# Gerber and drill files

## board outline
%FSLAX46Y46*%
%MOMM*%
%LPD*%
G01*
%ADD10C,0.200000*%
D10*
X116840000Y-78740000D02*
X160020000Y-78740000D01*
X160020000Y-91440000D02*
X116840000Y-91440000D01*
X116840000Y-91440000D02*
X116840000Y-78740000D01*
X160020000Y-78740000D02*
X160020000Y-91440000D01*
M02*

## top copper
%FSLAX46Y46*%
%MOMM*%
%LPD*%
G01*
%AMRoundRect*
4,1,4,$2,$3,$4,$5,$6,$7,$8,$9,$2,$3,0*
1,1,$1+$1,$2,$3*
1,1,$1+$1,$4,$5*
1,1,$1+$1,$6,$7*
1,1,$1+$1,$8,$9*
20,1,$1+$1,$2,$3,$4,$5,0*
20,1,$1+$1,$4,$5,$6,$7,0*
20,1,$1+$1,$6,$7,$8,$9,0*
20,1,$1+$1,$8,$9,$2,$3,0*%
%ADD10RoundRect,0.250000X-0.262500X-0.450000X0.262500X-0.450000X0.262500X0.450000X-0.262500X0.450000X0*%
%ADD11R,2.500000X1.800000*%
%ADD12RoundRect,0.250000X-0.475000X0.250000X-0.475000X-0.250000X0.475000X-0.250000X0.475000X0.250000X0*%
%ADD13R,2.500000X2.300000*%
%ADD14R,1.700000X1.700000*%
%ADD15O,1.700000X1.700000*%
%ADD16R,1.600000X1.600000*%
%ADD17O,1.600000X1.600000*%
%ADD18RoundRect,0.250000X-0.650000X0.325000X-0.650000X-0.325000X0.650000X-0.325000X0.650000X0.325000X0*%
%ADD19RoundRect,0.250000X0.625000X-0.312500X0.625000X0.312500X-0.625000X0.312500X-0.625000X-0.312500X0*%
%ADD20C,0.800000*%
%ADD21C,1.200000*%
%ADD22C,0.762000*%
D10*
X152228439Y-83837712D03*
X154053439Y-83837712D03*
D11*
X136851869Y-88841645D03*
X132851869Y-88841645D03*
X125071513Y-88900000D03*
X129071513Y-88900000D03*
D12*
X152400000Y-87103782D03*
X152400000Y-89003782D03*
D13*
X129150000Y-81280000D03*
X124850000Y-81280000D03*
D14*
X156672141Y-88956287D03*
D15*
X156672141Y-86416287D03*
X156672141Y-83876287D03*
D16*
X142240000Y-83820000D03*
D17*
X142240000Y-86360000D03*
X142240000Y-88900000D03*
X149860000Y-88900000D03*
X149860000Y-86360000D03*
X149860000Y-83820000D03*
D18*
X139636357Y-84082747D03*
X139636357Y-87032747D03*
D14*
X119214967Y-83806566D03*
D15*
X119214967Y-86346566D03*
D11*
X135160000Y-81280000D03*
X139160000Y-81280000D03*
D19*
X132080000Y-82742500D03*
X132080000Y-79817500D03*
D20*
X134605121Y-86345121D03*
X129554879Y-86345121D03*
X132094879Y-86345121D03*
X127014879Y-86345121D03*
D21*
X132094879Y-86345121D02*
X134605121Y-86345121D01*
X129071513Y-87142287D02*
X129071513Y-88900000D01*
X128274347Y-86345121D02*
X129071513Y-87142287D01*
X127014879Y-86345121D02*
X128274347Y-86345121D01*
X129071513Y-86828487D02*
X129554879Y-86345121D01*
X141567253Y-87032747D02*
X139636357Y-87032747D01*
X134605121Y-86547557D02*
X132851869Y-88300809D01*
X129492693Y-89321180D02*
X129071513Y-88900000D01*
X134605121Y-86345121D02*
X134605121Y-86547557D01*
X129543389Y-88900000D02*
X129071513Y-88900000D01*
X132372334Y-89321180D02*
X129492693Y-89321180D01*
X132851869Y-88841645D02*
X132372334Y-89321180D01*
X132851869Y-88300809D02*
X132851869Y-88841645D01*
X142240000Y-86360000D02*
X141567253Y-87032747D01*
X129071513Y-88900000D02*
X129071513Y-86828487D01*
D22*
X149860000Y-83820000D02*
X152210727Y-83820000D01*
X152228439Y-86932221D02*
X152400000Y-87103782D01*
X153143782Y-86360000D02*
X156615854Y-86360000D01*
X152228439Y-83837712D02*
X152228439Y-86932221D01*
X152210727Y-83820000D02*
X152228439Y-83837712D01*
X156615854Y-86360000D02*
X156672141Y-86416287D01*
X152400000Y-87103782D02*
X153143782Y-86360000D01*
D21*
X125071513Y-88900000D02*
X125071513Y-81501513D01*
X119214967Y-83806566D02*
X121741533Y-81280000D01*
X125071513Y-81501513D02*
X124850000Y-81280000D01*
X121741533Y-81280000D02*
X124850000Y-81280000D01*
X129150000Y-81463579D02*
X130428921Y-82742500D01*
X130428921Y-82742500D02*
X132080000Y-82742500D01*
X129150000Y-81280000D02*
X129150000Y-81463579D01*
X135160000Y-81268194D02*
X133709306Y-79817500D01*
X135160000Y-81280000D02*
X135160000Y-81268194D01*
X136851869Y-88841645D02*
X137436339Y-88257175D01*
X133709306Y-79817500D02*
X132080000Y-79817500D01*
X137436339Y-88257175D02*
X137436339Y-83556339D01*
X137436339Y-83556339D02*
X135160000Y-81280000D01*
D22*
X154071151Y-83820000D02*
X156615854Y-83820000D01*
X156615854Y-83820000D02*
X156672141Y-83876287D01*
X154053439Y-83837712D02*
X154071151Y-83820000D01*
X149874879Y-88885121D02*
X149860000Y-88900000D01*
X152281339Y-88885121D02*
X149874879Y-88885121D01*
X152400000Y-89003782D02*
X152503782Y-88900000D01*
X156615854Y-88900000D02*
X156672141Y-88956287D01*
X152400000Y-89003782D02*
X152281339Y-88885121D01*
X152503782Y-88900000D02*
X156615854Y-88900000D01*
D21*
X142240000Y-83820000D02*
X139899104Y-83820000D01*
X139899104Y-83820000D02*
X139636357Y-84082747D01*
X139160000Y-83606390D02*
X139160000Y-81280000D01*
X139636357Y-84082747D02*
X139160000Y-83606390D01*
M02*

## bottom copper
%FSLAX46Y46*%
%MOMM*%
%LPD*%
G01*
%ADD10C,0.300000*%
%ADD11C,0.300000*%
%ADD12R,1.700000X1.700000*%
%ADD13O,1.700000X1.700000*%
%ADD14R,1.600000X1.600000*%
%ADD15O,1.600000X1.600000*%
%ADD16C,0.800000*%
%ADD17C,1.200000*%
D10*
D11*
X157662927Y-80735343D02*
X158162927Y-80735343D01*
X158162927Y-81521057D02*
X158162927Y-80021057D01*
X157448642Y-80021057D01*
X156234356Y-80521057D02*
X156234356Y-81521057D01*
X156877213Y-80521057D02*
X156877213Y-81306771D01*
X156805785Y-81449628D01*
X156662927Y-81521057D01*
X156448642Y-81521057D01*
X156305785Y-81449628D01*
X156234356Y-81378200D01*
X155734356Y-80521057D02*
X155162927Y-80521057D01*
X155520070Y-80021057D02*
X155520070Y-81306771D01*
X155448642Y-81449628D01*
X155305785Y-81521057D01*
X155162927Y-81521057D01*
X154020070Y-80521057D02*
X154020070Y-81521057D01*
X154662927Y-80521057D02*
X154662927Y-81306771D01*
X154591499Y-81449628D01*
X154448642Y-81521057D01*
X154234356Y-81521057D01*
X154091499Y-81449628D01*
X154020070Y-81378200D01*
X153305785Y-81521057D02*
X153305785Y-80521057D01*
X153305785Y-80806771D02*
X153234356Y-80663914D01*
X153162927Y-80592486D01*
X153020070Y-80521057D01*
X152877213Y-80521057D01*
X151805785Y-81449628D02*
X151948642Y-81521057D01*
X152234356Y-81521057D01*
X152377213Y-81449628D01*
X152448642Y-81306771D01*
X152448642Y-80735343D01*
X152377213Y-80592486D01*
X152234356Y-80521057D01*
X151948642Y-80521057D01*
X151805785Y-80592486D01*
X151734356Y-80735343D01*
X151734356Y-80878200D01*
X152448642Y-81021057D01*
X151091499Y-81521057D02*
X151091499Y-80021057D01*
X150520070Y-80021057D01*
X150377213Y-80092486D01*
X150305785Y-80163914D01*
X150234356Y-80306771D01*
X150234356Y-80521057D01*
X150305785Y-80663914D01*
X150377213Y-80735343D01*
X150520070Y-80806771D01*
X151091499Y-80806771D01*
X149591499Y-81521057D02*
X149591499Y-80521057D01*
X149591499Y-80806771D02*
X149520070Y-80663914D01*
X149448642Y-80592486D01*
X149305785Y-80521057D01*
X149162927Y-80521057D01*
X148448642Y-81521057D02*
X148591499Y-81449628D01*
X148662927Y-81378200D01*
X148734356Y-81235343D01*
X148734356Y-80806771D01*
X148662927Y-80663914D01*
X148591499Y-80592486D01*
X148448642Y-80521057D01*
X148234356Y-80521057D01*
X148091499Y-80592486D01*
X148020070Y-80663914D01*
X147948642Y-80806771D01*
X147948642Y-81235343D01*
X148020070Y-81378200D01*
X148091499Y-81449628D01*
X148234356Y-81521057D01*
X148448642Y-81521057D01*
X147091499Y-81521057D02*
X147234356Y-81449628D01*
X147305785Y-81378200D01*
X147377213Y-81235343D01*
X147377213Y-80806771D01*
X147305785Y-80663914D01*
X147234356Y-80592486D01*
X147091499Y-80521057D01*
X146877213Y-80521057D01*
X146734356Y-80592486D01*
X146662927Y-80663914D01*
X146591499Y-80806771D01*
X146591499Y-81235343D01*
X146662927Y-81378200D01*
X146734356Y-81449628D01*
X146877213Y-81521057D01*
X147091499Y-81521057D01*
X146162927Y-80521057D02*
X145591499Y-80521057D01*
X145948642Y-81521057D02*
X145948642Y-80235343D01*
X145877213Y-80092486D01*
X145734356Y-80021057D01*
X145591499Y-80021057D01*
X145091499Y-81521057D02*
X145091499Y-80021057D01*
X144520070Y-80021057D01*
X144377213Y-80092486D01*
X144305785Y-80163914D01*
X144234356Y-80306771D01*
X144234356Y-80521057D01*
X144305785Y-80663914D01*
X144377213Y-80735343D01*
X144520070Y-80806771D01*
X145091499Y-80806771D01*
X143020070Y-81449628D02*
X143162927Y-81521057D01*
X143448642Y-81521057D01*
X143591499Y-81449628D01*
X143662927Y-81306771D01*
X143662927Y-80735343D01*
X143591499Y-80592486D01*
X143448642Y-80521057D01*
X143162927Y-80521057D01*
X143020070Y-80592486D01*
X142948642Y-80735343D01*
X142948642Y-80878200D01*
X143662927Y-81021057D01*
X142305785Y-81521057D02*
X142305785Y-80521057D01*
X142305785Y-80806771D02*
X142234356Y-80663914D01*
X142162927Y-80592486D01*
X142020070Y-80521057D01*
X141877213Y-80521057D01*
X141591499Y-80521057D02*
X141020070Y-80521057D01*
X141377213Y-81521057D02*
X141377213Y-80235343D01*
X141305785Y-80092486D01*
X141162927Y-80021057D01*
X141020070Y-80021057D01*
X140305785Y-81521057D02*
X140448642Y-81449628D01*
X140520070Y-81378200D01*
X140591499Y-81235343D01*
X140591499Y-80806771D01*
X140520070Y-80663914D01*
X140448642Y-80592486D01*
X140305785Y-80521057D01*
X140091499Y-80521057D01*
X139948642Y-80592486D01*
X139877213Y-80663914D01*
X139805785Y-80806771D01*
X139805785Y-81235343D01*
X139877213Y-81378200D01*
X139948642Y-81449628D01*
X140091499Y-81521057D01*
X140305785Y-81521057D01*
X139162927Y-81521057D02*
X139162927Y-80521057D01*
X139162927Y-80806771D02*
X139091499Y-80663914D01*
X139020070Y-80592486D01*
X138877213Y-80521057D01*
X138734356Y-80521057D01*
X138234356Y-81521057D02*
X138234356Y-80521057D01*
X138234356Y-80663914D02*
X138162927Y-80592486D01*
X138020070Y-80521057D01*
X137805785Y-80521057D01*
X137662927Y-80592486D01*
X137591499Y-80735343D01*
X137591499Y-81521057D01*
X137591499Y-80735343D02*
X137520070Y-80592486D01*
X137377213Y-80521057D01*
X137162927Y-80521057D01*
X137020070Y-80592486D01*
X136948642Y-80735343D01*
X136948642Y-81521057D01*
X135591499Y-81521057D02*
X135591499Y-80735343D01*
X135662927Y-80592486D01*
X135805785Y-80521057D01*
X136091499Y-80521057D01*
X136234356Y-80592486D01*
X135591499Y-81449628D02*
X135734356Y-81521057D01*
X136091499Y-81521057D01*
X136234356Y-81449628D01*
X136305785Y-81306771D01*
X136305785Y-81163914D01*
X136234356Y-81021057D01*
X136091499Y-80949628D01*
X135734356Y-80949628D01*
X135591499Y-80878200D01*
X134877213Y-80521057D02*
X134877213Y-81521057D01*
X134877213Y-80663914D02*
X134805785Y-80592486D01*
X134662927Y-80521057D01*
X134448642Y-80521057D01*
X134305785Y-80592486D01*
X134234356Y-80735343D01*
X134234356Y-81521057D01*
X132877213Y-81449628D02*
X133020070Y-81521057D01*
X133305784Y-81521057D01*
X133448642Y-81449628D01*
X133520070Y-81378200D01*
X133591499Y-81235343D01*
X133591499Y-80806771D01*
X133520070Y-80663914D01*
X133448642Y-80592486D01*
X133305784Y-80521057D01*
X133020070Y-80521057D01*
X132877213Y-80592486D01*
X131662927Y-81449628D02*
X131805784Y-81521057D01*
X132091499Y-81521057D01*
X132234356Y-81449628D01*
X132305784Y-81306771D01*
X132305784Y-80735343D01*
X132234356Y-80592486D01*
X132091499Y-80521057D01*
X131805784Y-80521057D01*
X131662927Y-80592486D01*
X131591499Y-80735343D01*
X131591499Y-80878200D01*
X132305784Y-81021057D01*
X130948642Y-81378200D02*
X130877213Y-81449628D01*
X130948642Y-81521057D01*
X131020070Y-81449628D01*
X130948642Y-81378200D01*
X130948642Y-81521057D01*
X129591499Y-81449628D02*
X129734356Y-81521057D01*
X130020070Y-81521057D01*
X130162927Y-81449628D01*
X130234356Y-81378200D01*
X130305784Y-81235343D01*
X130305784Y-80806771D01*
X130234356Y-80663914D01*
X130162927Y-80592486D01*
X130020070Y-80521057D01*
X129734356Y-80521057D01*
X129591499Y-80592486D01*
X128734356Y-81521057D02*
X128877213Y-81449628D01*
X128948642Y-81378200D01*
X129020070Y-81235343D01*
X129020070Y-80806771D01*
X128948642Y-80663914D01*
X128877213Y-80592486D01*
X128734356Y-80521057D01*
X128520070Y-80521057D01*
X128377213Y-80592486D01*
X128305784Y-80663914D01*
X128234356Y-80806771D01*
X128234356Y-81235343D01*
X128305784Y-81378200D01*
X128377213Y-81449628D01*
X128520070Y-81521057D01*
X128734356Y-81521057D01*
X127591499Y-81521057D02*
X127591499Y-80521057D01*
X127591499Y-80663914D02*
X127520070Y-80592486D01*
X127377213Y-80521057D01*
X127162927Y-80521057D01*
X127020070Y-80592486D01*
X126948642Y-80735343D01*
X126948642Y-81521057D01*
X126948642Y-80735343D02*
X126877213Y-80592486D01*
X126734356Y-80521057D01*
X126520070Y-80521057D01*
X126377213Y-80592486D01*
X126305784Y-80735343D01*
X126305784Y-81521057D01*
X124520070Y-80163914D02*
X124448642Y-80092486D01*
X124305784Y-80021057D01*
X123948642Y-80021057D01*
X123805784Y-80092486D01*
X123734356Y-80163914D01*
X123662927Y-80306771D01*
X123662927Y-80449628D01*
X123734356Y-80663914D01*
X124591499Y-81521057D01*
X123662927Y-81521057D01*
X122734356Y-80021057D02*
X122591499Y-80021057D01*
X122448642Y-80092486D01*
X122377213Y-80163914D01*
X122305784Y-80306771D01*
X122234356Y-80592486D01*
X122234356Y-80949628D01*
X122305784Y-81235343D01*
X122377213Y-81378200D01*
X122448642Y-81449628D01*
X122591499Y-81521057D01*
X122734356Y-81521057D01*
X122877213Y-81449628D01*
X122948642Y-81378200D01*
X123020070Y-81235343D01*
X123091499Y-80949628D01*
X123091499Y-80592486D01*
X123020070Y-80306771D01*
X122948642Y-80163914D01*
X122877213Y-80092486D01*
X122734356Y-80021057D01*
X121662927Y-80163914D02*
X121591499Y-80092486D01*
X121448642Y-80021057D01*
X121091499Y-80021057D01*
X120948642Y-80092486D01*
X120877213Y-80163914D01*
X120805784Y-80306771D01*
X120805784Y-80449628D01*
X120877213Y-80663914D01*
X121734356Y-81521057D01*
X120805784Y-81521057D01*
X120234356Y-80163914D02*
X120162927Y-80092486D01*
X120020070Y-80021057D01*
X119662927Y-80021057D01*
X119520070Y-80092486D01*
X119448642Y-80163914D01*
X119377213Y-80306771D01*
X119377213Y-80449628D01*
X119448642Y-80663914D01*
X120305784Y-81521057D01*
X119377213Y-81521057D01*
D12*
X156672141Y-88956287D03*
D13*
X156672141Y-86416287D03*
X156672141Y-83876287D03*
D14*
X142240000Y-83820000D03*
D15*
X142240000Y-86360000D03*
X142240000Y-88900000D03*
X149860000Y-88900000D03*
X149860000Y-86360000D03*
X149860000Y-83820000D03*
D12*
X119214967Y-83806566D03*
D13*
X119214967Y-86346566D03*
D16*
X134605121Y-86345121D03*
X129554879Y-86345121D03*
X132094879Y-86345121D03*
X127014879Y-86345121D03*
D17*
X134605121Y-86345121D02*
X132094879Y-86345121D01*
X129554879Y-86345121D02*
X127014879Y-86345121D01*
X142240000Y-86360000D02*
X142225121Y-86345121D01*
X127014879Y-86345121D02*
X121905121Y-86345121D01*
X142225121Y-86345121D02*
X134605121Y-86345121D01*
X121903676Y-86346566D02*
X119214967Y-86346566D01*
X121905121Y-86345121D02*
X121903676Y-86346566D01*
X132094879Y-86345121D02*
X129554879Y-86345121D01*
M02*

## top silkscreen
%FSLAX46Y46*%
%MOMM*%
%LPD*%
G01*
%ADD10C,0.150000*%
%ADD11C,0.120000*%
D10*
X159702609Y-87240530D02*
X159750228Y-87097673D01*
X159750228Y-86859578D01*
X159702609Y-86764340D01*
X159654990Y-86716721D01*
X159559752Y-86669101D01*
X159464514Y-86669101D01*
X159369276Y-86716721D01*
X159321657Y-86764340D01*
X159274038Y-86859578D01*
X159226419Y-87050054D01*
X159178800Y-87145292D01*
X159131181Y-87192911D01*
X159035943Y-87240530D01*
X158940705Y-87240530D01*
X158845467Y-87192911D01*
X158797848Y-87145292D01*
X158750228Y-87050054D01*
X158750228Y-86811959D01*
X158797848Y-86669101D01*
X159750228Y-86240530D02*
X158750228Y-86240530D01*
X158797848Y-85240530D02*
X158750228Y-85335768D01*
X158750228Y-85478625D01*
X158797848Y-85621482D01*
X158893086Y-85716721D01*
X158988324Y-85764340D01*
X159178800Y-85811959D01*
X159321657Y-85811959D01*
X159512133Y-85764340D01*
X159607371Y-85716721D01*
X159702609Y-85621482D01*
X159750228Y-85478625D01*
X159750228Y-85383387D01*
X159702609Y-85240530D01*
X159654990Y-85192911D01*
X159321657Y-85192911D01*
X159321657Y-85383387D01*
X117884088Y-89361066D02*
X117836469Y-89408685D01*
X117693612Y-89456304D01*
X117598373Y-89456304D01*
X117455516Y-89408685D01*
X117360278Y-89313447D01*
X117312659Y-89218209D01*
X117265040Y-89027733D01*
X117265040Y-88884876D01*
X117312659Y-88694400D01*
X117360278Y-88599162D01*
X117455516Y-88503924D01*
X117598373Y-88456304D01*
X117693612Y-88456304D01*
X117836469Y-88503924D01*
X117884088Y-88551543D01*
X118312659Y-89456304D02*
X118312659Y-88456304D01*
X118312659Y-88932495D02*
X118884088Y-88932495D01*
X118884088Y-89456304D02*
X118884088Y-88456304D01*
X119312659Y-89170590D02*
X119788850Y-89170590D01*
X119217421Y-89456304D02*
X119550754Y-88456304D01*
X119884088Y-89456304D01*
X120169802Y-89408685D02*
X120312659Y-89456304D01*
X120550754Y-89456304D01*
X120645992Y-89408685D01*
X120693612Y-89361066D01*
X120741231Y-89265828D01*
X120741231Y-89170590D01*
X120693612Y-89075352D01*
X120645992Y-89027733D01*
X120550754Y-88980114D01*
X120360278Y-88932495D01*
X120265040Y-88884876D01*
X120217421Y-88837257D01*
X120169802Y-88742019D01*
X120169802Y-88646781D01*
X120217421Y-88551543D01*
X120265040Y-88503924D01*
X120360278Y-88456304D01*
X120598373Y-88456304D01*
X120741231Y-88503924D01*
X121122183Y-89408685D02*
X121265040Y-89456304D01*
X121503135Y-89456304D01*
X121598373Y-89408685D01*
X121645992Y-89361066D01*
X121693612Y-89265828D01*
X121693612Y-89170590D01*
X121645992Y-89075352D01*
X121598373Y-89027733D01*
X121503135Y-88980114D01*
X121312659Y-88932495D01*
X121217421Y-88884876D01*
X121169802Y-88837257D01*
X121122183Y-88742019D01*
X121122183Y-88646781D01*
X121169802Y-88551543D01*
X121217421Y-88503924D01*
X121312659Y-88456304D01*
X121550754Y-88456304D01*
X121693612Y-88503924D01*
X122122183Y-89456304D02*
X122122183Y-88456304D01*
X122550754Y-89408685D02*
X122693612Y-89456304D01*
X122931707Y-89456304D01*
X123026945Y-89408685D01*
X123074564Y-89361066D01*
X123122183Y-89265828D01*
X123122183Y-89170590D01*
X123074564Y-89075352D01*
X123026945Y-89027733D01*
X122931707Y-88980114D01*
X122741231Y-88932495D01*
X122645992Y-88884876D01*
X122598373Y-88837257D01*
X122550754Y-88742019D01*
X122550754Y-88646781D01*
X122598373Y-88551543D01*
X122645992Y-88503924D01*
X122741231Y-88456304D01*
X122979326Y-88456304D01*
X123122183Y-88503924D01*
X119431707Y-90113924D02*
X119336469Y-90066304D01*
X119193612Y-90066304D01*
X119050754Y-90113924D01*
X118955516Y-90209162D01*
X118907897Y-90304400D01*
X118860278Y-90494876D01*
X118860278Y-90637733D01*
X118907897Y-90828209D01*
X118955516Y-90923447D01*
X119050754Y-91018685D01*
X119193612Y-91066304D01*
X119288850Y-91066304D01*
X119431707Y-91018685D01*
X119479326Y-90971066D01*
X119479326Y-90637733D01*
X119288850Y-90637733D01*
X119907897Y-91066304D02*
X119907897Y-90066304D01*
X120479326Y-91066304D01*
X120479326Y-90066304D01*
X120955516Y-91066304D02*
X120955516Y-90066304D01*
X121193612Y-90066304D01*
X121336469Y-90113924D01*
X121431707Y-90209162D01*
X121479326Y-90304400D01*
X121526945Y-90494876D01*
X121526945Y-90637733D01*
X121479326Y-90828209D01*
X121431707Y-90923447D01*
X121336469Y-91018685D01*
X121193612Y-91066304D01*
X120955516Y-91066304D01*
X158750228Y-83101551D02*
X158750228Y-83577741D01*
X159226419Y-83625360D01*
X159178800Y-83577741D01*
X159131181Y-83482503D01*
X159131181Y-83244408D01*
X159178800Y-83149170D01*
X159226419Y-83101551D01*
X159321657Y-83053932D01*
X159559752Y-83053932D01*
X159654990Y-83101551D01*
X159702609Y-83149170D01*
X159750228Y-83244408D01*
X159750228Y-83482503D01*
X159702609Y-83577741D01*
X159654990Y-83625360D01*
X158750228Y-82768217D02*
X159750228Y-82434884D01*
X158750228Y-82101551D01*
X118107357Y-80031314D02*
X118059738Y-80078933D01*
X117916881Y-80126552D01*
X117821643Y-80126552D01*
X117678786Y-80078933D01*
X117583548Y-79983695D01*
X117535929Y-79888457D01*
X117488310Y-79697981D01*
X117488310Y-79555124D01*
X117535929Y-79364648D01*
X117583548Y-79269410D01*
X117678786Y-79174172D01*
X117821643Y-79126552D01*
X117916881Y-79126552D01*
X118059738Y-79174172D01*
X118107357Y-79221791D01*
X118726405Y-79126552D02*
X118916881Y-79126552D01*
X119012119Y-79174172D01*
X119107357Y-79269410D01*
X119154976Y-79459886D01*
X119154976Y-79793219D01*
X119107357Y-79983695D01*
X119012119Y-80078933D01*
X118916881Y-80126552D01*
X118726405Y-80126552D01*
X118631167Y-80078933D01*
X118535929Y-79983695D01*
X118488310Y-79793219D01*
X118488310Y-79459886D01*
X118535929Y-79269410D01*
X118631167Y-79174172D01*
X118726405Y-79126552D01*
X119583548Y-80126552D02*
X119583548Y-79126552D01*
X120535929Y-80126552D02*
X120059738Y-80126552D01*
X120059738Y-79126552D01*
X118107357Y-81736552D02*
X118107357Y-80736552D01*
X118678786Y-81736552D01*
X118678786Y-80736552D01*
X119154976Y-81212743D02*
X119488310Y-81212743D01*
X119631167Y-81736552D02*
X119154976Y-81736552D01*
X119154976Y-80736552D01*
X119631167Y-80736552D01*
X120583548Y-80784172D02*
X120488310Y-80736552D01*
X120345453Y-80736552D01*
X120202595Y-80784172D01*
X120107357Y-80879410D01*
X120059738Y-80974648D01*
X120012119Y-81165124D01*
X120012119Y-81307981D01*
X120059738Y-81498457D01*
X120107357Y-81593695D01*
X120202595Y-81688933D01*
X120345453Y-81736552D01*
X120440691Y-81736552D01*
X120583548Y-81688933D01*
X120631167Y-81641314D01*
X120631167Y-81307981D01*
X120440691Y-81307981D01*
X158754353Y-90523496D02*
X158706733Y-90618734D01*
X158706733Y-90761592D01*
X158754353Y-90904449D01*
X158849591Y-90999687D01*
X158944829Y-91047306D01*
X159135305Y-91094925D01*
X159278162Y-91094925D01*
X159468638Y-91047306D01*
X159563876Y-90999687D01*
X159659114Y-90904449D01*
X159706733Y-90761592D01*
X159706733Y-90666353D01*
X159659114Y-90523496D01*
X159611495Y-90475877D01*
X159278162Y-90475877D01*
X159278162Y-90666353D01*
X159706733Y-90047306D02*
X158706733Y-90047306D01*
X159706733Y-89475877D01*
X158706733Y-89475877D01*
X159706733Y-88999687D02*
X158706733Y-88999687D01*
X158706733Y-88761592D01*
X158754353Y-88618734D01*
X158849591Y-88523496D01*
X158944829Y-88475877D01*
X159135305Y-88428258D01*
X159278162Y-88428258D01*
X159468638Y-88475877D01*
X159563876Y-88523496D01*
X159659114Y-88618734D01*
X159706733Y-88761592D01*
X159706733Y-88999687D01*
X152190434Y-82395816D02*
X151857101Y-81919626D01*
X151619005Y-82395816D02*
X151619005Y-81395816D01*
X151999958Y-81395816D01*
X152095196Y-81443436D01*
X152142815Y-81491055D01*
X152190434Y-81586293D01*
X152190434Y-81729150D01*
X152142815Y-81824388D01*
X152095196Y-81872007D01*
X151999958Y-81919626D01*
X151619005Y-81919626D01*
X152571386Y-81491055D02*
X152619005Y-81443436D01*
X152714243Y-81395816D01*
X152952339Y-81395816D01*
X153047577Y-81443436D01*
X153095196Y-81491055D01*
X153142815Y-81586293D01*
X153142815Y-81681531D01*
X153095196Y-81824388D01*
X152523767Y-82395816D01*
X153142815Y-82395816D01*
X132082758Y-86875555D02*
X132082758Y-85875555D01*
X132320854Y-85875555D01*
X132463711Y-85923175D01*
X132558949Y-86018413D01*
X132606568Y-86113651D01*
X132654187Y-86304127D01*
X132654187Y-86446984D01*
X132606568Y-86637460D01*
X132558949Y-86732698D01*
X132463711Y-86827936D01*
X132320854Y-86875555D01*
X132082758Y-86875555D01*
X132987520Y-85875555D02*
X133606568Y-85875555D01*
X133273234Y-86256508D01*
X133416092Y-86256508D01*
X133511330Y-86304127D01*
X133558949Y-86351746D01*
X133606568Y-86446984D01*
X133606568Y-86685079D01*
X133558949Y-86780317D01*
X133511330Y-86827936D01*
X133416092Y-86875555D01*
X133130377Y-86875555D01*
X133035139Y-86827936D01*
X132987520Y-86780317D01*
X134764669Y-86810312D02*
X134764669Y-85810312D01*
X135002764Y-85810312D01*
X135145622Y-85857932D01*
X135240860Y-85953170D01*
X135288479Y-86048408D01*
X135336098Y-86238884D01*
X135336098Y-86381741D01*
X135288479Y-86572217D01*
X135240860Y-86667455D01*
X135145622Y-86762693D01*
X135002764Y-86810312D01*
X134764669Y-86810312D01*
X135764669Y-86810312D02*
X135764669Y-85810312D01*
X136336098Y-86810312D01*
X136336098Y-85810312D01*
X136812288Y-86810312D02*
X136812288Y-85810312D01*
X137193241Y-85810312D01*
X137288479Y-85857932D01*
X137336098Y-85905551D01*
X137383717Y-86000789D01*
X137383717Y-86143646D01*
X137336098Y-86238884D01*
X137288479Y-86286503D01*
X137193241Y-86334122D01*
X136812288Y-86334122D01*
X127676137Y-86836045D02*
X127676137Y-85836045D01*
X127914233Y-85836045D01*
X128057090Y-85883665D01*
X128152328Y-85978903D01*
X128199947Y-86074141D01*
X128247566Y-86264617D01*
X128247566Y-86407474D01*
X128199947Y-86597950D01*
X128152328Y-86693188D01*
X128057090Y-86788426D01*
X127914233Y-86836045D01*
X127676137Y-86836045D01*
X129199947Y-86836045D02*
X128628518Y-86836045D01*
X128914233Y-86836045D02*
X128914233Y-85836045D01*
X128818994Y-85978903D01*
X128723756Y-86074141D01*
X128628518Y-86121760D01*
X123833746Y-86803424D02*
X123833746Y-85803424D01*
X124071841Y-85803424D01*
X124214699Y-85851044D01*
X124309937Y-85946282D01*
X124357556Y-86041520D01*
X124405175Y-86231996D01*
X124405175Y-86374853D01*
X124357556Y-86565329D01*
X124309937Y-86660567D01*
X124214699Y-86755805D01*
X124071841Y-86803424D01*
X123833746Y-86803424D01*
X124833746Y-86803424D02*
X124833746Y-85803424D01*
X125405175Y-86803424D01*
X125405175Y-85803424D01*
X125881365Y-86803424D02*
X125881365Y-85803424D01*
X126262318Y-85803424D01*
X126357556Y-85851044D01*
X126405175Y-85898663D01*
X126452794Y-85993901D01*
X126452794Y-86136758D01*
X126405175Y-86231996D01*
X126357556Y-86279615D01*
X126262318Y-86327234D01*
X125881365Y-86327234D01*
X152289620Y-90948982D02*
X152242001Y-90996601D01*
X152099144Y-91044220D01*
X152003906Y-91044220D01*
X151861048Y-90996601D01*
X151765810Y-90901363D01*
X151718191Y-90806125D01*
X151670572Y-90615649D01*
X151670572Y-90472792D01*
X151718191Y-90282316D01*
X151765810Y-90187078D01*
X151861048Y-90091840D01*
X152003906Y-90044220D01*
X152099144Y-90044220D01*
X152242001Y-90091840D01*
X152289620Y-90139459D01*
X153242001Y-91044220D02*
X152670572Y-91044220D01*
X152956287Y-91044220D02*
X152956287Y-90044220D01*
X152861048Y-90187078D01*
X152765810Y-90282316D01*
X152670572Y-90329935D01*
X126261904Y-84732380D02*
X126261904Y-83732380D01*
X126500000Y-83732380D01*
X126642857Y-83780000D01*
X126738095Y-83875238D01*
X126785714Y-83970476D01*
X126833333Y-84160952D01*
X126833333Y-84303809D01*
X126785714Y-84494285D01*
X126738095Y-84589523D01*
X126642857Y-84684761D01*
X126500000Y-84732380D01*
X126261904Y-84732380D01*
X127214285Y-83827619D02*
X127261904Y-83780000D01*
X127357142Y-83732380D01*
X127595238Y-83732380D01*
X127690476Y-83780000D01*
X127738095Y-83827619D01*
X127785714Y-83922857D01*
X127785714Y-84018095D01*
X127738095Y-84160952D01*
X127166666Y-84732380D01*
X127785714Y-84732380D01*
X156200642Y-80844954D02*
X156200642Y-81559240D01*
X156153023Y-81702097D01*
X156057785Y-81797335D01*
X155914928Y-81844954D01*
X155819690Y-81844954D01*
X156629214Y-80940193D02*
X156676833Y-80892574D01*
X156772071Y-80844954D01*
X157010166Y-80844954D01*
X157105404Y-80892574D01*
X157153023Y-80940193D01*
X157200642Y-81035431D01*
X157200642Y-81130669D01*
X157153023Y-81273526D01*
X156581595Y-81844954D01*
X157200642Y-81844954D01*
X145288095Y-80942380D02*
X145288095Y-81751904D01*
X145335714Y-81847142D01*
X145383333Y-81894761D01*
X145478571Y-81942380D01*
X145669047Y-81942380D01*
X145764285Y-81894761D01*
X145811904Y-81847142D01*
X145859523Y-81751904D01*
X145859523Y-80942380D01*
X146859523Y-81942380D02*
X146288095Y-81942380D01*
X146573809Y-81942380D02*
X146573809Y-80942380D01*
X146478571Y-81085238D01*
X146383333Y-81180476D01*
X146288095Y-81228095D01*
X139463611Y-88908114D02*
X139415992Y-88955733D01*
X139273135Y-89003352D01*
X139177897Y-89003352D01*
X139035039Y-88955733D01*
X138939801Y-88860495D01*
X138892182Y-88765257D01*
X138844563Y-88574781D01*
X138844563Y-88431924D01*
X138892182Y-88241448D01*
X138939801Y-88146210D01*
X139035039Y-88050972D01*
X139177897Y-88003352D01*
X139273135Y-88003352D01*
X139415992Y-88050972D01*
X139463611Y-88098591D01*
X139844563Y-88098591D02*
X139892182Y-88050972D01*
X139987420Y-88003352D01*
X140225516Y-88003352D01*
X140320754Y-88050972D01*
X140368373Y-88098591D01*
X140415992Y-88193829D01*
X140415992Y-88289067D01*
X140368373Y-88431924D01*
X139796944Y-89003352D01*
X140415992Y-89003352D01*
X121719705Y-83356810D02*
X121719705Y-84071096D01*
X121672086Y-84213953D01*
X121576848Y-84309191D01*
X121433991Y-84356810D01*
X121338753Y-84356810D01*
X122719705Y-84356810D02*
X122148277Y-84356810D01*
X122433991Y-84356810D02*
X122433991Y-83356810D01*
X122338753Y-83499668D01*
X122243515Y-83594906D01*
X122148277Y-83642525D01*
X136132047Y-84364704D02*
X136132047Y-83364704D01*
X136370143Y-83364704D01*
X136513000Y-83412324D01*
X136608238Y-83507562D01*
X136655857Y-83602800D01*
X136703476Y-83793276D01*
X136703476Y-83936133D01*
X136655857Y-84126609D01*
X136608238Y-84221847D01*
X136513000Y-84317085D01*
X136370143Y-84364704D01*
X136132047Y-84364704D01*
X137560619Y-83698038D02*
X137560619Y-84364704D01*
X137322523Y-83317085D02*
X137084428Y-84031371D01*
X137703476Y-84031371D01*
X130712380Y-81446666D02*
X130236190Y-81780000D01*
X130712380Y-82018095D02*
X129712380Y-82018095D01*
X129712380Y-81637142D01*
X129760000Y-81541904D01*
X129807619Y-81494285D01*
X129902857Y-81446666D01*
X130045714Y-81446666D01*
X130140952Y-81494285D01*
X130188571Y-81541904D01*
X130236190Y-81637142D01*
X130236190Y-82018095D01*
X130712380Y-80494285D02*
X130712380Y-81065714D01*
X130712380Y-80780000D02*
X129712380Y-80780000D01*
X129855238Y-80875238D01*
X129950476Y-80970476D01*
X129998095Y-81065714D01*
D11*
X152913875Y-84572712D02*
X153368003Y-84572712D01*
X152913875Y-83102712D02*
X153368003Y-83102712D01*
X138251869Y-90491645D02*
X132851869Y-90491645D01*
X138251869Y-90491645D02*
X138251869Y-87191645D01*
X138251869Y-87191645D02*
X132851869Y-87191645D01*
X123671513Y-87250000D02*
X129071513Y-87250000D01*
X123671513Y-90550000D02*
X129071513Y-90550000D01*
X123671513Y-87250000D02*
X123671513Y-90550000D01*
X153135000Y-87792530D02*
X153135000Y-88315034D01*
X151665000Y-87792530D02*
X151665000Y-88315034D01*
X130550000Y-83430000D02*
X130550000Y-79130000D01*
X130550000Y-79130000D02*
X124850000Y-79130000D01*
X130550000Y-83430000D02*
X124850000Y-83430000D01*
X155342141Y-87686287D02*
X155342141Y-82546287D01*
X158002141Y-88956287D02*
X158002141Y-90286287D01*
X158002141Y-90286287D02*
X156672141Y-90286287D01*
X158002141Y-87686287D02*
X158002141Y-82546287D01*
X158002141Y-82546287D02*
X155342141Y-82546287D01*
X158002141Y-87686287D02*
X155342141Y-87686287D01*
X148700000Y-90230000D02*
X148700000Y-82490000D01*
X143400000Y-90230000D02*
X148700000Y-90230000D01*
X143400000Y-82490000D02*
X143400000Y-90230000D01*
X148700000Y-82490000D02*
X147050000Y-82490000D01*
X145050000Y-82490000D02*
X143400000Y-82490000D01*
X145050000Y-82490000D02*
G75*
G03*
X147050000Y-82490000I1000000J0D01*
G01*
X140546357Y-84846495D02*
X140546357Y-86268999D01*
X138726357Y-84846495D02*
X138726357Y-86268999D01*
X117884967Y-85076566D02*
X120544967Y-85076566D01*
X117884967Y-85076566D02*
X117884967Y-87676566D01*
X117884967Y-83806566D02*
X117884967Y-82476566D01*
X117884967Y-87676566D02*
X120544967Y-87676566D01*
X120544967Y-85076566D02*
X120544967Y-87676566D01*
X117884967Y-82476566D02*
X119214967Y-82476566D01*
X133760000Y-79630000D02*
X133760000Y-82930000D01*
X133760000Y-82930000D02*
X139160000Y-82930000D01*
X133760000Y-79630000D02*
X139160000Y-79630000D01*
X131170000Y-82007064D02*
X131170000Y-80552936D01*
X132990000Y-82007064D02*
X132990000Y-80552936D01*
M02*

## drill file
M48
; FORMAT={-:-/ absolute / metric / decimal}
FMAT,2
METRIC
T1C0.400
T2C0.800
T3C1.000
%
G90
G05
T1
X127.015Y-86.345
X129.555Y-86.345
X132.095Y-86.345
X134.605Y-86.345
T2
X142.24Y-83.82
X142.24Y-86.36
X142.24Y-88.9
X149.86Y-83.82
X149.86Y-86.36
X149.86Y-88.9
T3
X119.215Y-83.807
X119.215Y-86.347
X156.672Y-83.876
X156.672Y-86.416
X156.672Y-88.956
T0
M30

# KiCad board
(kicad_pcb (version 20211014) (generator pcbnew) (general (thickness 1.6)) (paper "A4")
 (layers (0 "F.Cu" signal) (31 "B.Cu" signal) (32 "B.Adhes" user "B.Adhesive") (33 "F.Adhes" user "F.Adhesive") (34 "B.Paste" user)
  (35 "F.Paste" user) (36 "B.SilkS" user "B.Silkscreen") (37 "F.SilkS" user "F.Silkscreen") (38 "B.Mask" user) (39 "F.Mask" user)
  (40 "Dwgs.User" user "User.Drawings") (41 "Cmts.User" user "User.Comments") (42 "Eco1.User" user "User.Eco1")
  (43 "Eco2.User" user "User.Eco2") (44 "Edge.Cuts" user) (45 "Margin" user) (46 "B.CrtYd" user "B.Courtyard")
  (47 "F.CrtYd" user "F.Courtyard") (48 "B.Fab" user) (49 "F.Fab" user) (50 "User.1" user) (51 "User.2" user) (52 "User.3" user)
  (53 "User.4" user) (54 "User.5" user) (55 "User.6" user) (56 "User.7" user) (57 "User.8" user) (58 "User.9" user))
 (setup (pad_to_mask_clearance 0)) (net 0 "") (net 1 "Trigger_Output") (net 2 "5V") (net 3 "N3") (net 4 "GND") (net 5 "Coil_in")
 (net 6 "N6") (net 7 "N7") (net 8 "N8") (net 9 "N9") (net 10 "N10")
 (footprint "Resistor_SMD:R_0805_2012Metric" (layer "F.Cu") (at 153.140939 83.837712)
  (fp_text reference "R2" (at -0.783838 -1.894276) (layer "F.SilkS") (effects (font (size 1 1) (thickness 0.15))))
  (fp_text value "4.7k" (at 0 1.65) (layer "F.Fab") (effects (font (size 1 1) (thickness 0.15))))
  (fp_line (start -0.227064 0.735) (end 0.227064 0.735) (layer "F.SilkS") (width 0.12))
  (fp_line (start -0.227064 -0.735) (end 0.227064 -0.735) (layer "F.SilkS") (width 0.12))
  (pad "1" smd roundrect (at -0.9125 0) (size 1.025 1.4) (layers "F.Cu" "F.Paste" "F.Mask") (roundrect_rratio 0.243902439)
   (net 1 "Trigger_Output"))
  (pad "2" smd roundrect (at 0.9125 0) (size 1.025 1.4) (layers "F.Cu" "F.Paste" "F.Mask") (roundrect_rratio 0.243902439) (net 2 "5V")))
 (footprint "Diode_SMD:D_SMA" (layer "F.Cu") (at 134.851869 88.841645 180)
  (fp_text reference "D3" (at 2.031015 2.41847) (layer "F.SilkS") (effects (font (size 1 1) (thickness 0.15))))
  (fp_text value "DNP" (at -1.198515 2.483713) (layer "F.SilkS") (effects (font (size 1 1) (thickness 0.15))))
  (fp_line (start -3.4 -1.65) (end 2 -1.65) (layer "F.SilkS") (width 0.12))
  (fp_line (start -3.4 -1.65) (end -3.4 1.65) (layer "F.SilkS") (width 0.12))
  (fp_line (start -3.4 1.65) (end 2 1.65) (layer "F.SilkS") (width 0.12))
  (pad "1" smd rect (at -2 0 180) (size 2.5 1.8) (layers "F.Cu" "F.Paste" "F.Mask") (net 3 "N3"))
  (pad "2" smd rect (at 2 0 180) (size 2.5 1.8) (layers "F.Cu" "F.Paste" "F.Mask") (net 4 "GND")))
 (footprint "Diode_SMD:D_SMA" (layer "F.Cu") (at 127.071513 88.9)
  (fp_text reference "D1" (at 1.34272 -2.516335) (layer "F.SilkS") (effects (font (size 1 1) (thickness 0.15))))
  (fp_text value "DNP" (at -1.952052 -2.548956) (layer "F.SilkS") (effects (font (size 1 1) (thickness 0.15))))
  (fp_line (start -3.4 -1.65) (end 2 -1.65) (layer "F.SilkS") (width 0.12))
  (fp_line (start -3.4 1.65) (end 2 1.65) (layer "F.SilkS") (width 0.12))
  (fp_line (start -3.4 -1.65) (end -3.4 1.65) (layer "F.SilkS") (width 0.12))
  (pad "1" smd rect (at -2 0) (size 2.5 1.8) (layers "F.Cu" "F.Paste" "F.Mask") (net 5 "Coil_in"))
  (pad "2" smd rect (at 2 0) (size 2.5 1.8) (layers "F.Cu" "F.Paste" "F.Mask") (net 4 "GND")))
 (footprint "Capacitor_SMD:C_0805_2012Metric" (layer "F.Cu") (at 152.4 88.053782 -90)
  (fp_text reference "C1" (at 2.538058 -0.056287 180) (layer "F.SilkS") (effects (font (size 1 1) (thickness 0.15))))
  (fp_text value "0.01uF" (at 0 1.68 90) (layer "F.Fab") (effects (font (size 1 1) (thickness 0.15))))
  (fp_line (start -0.261252 -0.735) (end 0.261252 -0.735) (layer "F.SilkS") (width 0.12))
  (fp_line (start -0.261252 0.735) (end 0.261252 0.735) (layer "F.SilkS") (width 0.12))
  (pad "1" smd roundrect (at -0.95 0 270) (size 1 1.45) (layers "F.Cu" "F.Paste" "F.Mask") (roundrect_rratio 0.25) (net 1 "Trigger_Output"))
  (pad "2" smd roundrect (at 0.95 0 270) (size 1 1.45) (layers "F.Cu" "F.Paste" "F.Mask") (roundrect_rratio 0.25) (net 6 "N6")))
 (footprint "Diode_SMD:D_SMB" (layer "F.Cu") (at 127 81.28 180)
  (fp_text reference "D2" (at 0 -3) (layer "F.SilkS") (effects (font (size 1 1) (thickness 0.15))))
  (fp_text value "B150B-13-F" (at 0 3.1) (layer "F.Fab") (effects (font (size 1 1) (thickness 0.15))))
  (fp_line (start -3.55 -2.15) (end -3.55 2.15) (layer "F.SilkS") (width 0.12))
  (fp_line (start -3.55 2.15) (end 2.15 2.15) (layer "F.SilkS") (width 0.12))
  (fp_line (start -3.55 -2.15) (end 2.15 -2.15) (layer "F.SilkS") (width 0.12))
  (pad "1" smd rect (at -2.15 0 180) (size 2.5 2.3) (layers "F.Cu" "F.Paste" "F.Mask") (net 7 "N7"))
  (pad "2" smd rect (at 2.15 0 180) (size 2.5 2.3) (layers "F.Cu" "F.Paste" "F.Mask") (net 5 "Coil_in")))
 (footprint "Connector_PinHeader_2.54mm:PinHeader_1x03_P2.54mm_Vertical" (layer "F.Cu") (at 156.672141 88.956287 180)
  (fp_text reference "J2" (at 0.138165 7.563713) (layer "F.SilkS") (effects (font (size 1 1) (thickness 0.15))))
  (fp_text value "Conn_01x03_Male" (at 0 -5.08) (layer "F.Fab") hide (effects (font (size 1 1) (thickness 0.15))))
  (fp_line (start 1.33 1.27) (end 1.33 6.41) (layer "F.SilkS") (width 0.12))
  (fp_line (start -1.33 0) (end -1.33 -1.33) (layer "F.SilkS") (width 0.12))
  (fp_line (start -1.33 -1.33) (end 0 -1.33) (layer "F.SilkS") (width 0.12))
  (fp_line (start -1.33 1.27) (end -1.33 6.41) (layer "F.SilkS") (width 0.12))
  (fp_line (start -1.33 6.41) (end 1.33 6.41) (layer "F.SilkS") (width 0.12))
  (fp_line (start -1.33 1.27) (end 1.33 1.27) (layer "F.SilkS") (width 0.12))
  (pad "1" thru_hole rect (at 0 0 180) (size 1.7 1.7) (drill 1) (layers *.Cu *.Mask) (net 6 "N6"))
  (pad "2" thru_hole oval (at 0 2.54 180) (size 1.7 1.7) (drill 1) (layers *.Cu *.Mask) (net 1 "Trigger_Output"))
  (pad "3" thru_hole oval (at 0 5.08 180) (size 1.7 1.7) (drill 1) (layers *.Cu *.Mask) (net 2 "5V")))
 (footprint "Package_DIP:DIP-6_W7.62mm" (layer "F.Cu") (at 142.24 83.82)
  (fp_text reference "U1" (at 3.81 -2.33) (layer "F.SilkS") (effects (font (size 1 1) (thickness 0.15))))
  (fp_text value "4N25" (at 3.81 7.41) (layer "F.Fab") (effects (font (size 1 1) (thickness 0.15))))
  (fp_line (start 6.46 6.41) (end 6.46 -1.33) (layer "F.SilkS") (width 0.12))
  (fp_line (start 1.16 6.41) (end 6.46 6.41) (layer "F.SilkS") (width 0.12))
  (fp_line (start 1.16 -1.33) (end 1.16 6.41) (layer "F.SilkS") (width 0.12))
  (fp_line (start 6.46 -1.33) (end 4.81 -1.33) (layer "F.SilkS") (width 0.12))
  (fp_line (start 2.81 -1.33) (end 1.16 -1.33) (layer "F.SilkS") (width 0.12))
  (fp_arc (start 4.81 -1.33) (mid 3.81 -0.33) (end 2.81 -1.33) (layer "F.SilkS") (width 0.12))
  (pad "1" thru_hole rect (at 0 0) (size 1.6 1.6) (drill 0.8) (layers *.Cu *.Mask) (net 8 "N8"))
  (pad "2" thru_hole oval (at 0 2.54) (size 1.6 1.6) (drill 0.8) (layers *.Cu *.Mask) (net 4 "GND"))
  (pad "3" thru_hole oval (at 0 5.08) (size 1.6 1.6) (drill 0.8) (layers *.Cu *.Mask) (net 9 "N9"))
  (pad "4" thru_hole oval (at 7.62 5.08) (size 1.6 1.6) (drill 0.8) (layers *.Cu *.Mask) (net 6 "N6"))
  (pad "5" thru_hole oval (at 7.62 2.54) (size 1.6 1.6) (drill 0.8) (layers *.Cu *.Mask) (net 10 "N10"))
  (pad "6" thru_hole oval (at 7.62 0) (size 1.6 1.6) (drill 0.8) (layers *.Cu *.Mask) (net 1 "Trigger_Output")))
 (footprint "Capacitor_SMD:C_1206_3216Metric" (layer "F.Cu") (at 139.636357 85.557747 -90)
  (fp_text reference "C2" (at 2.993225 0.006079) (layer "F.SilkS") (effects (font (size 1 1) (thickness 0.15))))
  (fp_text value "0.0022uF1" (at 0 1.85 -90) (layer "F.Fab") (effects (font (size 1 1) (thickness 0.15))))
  (fp_line (start -0.711252 -0.91) (end 0.711252 -0.91) (layer "F.SilkS") (width 0.12))
  (fp_line (start -0.711252 0.91) (end 0.711252 0.91) (layer "F.SilkS") (width 0.12))
  (pad "1" smd roundrect (at -1.475 0 270) (size 1.15 1.8) (layers "F.Cu" "F.Paste" "F.Mask") (roundrect_rratio 0.2173913043) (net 8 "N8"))
  (pad "2" smd roundrect (at 1.475 0 270) (size 1.15 1.8) (layers "F.Cu" "F.Paste" "F.Mask") (roundrect_rratio 0.2173913043) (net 4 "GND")))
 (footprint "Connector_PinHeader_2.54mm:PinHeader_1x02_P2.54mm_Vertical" (layer "F.Cu") (at 119.214967 83.806566)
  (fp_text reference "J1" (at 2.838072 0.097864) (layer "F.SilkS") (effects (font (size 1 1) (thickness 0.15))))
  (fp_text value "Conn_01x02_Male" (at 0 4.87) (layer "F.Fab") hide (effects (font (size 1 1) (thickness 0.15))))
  (fp_line (start -1.33 1.27) (end 1.33 1.27) (layer "F.SilkS") (width 0.12))
  (fp_line (start -1.33 1.27) (end -1.33 3.87) (layer "F.SilkS") (width 0.12))
  (fp_line (start -1.33 0) (end -1.33 -1.33) (layer "F.SilkS") (width 0.12))
  (fp_line (start -1.33 3.87) (end 1.33 3.87) (layer "F.SilkS") (width 0.12))
  (fp_line (start 1.33 1.27) (end 1.33 3.87) (layer "F.SilkS") (width 0.12))
  (fp_line (start -1.33 -1.33) (end 0 -1.33) (layer "F.SilkS") (width 0.12))
  (pad "1" thru_hole rect (at 0 0) (size 1.7 1.7) (drill 1) (layers *.Cu *.Mask) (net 5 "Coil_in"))
  (pad "2" thru_hole oval (at 0 2.54) (size 1.7 1.7) (drill 1) (layers *.Cu *.Mask) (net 4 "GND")))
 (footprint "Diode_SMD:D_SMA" (layer "F.Cu") (at 137.16 81.28)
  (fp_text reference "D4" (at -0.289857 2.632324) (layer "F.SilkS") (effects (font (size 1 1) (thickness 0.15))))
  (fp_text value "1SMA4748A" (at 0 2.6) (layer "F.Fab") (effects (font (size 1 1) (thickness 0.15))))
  (fp_line (start -3.4 -1.65) (end -3.4 1.65) (layer "F.SilkS") (width 0.12))
  (fp_line (start -3.4 1.65) (end 2 1.65) (layer "F.SilkS") (width 0.12))
  (fp_line (start -3.4 -1.65) (end 2 -1.65) (layer "F.SilkS") (width 0.12))
  (pad "1" smd rect (at -2 0) (size 2.5 1.8) (layers "F.Cu" "F.Paste" "F.Mask") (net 3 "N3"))
  (pad "2" smd rect (at 2 0) (size 2.5 1.8) (layers "F.Cu" "F.Paste" "F.Mask") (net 8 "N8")))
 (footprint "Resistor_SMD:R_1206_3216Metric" (layer "F.Cu") (at 132.08 81.28 90)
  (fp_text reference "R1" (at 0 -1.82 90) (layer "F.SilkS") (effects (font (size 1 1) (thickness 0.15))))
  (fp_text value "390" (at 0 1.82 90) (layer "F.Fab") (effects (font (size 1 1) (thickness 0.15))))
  (fp_line (start -0.727064 -0.91) (end 0.727064 -0.91) (layer "F.SilkS") (width 0.12))
  (fp_line (start -0.727064 0.91) (end 0.727064 0.91) (layer "F.SilkS") (width 0.12))
  (pad "1" smd roundrect (at -1.4625 0 90) (size 1.125 1.75) (layers "F.Cu" "F.Paste" "F.Mask") (roundrect_rratio 0.2222222222) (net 7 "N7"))
  (pad "2" smd roundrect (at 1.4625 0 90) (size 1.125 1.75) (layers "F.Cu" "F.Paste" "F.Mask") (roundrect_rratio 0.2222222222) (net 3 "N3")))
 (gr_line (start 116.84 78.74) (end 160.02 78.74) (layer "Edge.Cuts") (width 0.2))
 (gr_line (start 160.02 91.44) (end 116.84 91.44) (layer "Edge.Cuts") (width 0.2))
 (gr_line (start 116.84 91.44) (end 116.84 78.74) (layer "Edge.Cuts") (width 0.2))
 (gr_line (start 160.02 78.74) (end 160.02 91.44) (layer "Edge.Cuts") (width 0.2))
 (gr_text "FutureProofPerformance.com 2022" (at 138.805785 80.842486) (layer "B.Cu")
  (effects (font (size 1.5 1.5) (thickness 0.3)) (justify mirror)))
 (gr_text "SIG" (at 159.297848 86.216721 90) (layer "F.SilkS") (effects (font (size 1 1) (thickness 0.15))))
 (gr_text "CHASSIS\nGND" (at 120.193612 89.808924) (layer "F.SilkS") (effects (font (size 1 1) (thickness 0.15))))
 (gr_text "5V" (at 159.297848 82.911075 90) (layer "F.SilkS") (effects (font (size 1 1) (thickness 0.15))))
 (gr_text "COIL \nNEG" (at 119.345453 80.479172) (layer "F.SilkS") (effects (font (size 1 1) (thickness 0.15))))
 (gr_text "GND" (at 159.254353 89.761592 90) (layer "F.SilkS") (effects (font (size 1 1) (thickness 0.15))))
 (segment (start 129.071513 87.142287) (end 129.071513 88.9) (width 1.2) (layer "F.Cu") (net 4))
 (segment (start 129.071513 86.828487) (end 129.554879 86.345121) (width 1.2) (layer "F.Cu") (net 4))
 (segment (start 141.567253 87.032747) (end 139.636357 87.032747) (width 1.2) (layer "F.Cu") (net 4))
 (segment (start 134.605121 86.547557) (end 132.851869 88.300809) (width 1.2) (layer "F.Cu") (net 4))
 (segment (start 129.492693 89.32118) (end 129.071513 88.9) (width 1.2) (layer "F.Cu") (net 4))
 (segment (start 132.094879 86.345121) (end 134.605121 86.345121) (width 1.2) (layer "F.Cu") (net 4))
 (segment (start 134.605121 86.345121) (end 134.605121 86.547557) (width 1.2) (layer "F.Cu") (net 4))
 (segment (start 128.274347 86.345121) (end 129.071513 87.142287) (width 1.2) (layer "F.Cu") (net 4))
 (segment (start 129.543389 88.9) (end 129.071513 88.9) (width 1.2) (layer "F.Cu") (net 4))
 (segment (start 132.372334 89.32118) (end 129.492693 89.32118) (width 1.2) (layer "F.Cu") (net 4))
 (segment (start 132.851869 88.841645) (end 132.372334 89.32118) (width 1.2) (layer "F.Cu") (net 4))
 (segment (start 127.014879 86.345121) (end 128.274347 86.345121) (width 1.2) (layer "F.Cu") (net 4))
 (segment (start 132.851869 88.300809) (end 132.851869 88.841645) (width 1.2) (layer "F.Cu") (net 4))
 (segment (start 142.24 86.36) (end 141.567253 87.032747) (width 1.2) (layer "F.Cu") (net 4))
 (segment (start 129.071513 88.9) (end 129.071513 86.828487) (width 1.2) (layer "F.Cu") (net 4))
 (via (at 134.605121 86.345121) (size 0.8) (drill 0.4) (layers "F.Cu" "B.Cu") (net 4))
 (via (at 129.554879 86.345121) (size 0.8) (drill 0.4) (layers "F.Cu" "B.Cu") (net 4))
 (via (at 132.094879 86.345121) (size 0.8) (drill 0.4) (layers "F.Cu" "B.Cu") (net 4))
 (via (at 127.014879 86.345121) (size 0.8) (drill 0.4) (layers "F.Cu" "B.Cu") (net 4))
 (segment (start 142.24 86.36) (end 142.225121 86.345121) (width 1.2) (layer "B.Cu") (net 4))
 (segment (start 127.014879 86.345121) (end 121.905121 86.345121) (width 1.2) (layer "B.Cu") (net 4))
 (segment (start 142.225121 86.345121) (end 134.605121 86.345121) (width 1.2) (layer "B.Cu") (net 4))
 (segment (start 134.605121 86.345121) (end 132.094879 86.345121) (width 1.2) (layer "B.Cu") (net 4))
 (segment (start 121.903676 86.346566) (end 119.214967 86.346566) (width 1.2) (layer "B.Cu") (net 4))
 (segment (start 121.905121 86.345121) (end 121.903676 86.346566) (width 1.2) (layer "B.Cu") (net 4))
 (segment (start 132.094879 86.345121) (end 129.554879 86.345121) (width 1.2) (layer "B.Cu") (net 4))
 (segment (start 129.554879 86.345121) (end 127.014879 86.345121) (width 1.2) (layer "B.Cu") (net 4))
 (segment (start 149.86 83.82) (end 152.210727 83.82) (width 0.762) (layer "F.Cu") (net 1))
 (segment (start 152.228439 86.932221) (end 152.4 87.103782) (width 0.762) (layer "F.Cu") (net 1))
 (segment (start 153.143782 86.36) (end 156.615854 86.36) (width 0.762) (layer "F.Cu") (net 1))
 (segment (start 152.228439 83.837712) (end 152.228439 86.932221) (width 0.762) (layer "F.Cu") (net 1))
 (segment (start 152.210727 83.82) (end 152.228439 83.837712) (width 0.762) (layer "F.Cu") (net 1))
 (segment (start 156.615854 86.36) (end 156.672141 86.416287) (width 0.762) (layer "F.Cu") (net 1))
 (segment (start 152.4 87.103782) (end 153.143782 86.36) (width 0.762) (layer "F.Cu") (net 1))
 (segment (start 125.071513 88.9) (end 125.071513 81.501513) (width 1.2) (layer "F.Cu") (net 5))
 (segment (start 119.214967 83.806566) (end 121.741533 81.28) (width 1.2) (layer "F.Cu") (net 5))
 (segment (start 125.071513 81.501513) (end 124.85 81.28) (width 1.2) (layer "F.Cu") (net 5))
 (segment (start 121.741533 81.28) (end 124.85 81.28) (width 1.2) (layer "F.Cu") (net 5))
 (segment (start 129.15 81.463579) (end 130.428921 82.7425) (width 1.2) (layer "F.Cu") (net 7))
 (segment (start 130.428921 82.7425) (end 132.08 82.7425) (width 1.2) (layer "F.Cu") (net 7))
 (segment (start 129.15 81.28) (end 129.15 81.463579) (width 1.2) (layer "F.Cu") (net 7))
 (segment (start 135.16 81.268194) (end 133.709306 79.8175) (width 1.2) (layer "F.Cu") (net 3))
 (segment (start 135.16 81.28) (end 135.16 81.268194) (width 1.2) (layer "F.Cu") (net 3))
 (segment (start 136.851869 88.841645) (end 137.436339 88.257175) (width 1.2) (layer "F.Cu") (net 3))
 (segment (start 133.709306 79.8175) (end 132.08 79.8175) (width 1.2) (layer "F.Cu") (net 3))
 (segment (start 137.436339 88.257175) (end 137.436339 83.556339) (width 1.2) (layer "F.Cu") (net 3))
 (segment (start 137.436339 83.556339) (end 135.16 81.28) (width 1.2) (layer "F.Cu") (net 3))
 (segment (start 154.071151 83.82) (end 156.615854 83.82) (width 0.762) (layer "F.Cu") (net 2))
 (segment (start 156.615854 83.82) (end 156.672141 83.876287) (width 0.762) (layer "F.Cu") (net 2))
 (segment (start 154.053439 83.837712) (end 154.071151 83.82) (width 0.762) (layer "F.Cu") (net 2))
 (segment (start 149.874879 88.885121) (end 149.86 88.9) (width 0.762) (layer "F.Cu") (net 6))
 (segment (start 152.281339 88.885121) (end 149.874879 88.885121) (width 0.762) (layer "F.Cu") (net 6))
 (segment (start 152.4 89.003782) (end 152.503782 88.9) (width 0.762) (layer "F.Cu") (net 6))
 (segment (start 156.615854 88.9) (end 156.672141 88.956287) (width 0.762) (layer "F.Cu") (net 6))
 (segment (start 152.4 89.003782) (end 152.281339 88.885121) (width 0.762) (layer "F.Cu") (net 6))
 (segment (start 152.503782 88.9) (end 156.615854 88.9) (width 0.762) (layer "F.Cu") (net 6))
 (segment (start 142.24 83.82) (end 139.899104 83.82) (width 1.2) (layer "F.Cu") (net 8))
 (segment (start 139.899104 83.82) (end 139.636357 84.082747) (width 1.2) (layer "F.Cu") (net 8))
 (segment (start 139.16 83.60639) (end 139.16 81.28) (width 1.2) (layer "F.Cu") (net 8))
 (segment (start 139.636357 84.082747) (end 139.16 83.60639) (width 1.2) (layer "F.Cu") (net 8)))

